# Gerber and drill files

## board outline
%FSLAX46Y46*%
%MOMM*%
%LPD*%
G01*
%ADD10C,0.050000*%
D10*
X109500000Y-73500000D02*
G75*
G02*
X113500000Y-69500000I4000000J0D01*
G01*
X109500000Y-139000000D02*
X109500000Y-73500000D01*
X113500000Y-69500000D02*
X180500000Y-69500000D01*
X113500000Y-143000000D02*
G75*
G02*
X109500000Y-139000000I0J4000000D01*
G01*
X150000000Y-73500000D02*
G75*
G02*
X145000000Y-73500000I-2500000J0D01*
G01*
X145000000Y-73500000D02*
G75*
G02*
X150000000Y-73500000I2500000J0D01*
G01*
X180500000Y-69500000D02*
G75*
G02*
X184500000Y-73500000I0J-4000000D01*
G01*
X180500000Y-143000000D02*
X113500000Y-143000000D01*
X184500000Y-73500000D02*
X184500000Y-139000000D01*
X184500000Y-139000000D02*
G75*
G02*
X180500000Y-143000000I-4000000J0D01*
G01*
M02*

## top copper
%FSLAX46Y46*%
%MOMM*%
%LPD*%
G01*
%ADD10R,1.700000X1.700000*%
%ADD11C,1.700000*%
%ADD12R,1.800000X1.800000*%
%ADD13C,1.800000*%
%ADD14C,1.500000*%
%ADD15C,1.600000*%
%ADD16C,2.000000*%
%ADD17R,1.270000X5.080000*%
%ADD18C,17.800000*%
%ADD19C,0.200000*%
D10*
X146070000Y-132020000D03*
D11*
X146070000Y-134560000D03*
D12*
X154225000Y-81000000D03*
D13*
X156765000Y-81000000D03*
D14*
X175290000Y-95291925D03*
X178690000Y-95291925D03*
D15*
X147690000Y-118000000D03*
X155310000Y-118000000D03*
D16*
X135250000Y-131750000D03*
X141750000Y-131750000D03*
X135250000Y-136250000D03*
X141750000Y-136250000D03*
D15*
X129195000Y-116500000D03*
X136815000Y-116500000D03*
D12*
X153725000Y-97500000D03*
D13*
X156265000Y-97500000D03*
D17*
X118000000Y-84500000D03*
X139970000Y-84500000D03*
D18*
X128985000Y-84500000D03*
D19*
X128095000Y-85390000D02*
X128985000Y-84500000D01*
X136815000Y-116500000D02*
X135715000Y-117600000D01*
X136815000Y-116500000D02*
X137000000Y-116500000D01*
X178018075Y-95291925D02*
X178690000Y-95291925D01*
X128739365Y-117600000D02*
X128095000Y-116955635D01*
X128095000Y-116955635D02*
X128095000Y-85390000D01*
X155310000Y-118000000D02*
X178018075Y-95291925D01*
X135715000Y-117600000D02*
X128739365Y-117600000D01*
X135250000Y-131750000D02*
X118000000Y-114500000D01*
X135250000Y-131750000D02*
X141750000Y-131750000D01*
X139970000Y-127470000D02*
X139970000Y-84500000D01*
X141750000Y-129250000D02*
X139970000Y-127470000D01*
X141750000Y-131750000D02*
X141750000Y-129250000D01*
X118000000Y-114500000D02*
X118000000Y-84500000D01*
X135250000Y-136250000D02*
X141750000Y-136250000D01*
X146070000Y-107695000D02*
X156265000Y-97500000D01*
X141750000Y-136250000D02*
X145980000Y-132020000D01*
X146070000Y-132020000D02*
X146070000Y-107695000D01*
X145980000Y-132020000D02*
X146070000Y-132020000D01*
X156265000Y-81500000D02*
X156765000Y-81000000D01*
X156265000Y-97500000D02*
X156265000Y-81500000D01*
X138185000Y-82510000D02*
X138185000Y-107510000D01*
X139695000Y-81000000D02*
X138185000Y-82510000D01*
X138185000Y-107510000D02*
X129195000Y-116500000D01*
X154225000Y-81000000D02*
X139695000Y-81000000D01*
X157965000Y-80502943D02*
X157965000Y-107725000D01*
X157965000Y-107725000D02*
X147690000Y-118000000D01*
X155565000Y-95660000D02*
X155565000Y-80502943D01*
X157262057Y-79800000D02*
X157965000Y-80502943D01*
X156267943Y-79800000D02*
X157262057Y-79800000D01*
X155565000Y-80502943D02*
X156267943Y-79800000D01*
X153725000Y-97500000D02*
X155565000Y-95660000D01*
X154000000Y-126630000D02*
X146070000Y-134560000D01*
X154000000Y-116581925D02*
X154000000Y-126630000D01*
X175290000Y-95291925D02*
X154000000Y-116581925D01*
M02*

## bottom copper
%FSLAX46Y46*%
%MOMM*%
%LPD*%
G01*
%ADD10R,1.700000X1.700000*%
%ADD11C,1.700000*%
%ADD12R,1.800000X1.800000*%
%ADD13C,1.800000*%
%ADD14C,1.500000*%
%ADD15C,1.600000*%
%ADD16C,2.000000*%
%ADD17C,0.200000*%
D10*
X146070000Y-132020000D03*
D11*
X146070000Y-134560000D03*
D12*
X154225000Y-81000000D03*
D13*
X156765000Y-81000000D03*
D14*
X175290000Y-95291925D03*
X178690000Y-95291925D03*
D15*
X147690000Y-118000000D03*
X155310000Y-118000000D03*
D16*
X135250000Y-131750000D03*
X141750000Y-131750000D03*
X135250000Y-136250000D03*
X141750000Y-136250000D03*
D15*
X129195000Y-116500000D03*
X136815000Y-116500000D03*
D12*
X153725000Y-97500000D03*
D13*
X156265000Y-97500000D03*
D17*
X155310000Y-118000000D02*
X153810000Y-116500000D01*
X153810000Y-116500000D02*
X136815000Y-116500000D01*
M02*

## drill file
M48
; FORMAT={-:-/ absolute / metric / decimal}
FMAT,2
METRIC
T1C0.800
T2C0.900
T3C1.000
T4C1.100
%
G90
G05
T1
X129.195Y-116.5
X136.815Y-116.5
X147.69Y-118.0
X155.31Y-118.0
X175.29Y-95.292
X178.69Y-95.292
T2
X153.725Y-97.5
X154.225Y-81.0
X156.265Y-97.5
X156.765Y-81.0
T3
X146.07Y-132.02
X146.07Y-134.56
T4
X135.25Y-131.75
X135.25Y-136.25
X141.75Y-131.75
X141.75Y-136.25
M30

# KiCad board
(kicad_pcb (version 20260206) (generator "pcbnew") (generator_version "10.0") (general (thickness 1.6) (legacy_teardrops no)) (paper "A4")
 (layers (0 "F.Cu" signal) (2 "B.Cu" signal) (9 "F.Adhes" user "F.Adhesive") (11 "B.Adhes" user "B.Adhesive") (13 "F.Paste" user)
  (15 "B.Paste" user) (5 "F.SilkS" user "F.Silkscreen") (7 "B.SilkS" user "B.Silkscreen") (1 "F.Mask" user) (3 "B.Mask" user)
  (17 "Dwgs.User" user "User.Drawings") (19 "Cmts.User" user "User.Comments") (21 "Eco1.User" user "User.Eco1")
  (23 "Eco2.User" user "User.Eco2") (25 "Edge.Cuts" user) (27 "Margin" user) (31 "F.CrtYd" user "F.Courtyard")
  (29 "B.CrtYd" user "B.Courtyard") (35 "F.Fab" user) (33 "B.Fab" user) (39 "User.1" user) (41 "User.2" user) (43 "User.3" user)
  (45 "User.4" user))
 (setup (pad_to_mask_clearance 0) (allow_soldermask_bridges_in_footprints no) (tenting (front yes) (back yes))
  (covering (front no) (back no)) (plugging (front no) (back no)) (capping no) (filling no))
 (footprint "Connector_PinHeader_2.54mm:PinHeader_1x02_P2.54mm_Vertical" (layer "F.Cu") (at 146.07 132.02)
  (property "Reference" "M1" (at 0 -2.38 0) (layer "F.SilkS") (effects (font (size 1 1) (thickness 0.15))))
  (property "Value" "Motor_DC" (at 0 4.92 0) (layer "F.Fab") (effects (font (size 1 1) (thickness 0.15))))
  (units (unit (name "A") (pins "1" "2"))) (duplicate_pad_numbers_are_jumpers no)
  (pad "1" thru_hole rect (at 0 0) (size 1.7 1.7) (drill 1) (layers "*.Cu" "*.Mask") (remove_unused_layers no) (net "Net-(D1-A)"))
  (pad "2" thru_hole circle (at 0 2.54) (size 1.7 1.7) (drill 1) (layers "*.Cu" "*.Mask") (remove_unused_layers no) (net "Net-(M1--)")))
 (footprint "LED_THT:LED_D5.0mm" (layer "F.Cu") (at 154.225 81)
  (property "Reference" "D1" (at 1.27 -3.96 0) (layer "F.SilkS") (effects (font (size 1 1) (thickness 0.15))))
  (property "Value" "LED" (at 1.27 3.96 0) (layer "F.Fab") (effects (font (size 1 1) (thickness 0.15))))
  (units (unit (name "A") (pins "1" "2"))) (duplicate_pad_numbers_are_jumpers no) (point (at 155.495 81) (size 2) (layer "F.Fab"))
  (pad "1" thru_hole rect (at 0 0) (size 1.8 1.8) (drill 0.9) (layers "*.Cu" "*.Mask") (remove_unused_layers no) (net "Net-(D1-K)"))
  (pad "2" thru_hole circle (at 2.54 0) (size 1.8 1.8) (drill 0.9) (layers "*.Cu" "*.Mask") (remove_unused_layers no) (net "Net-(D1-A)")))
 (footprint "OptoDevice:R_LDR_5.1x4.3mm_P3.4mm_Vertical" (layer "F.Cu") (at 175.29 95.291925)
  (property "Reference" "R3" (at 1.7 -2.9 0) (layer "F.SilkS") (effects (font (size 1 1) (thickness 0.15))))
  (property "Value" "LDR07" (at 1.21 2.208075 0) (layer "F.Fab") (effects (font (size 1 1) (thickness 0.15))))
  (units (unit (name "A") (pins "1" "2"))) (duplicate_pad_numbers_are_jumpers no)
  (pad "1" thru_hole circle (at 0 0) (size 1.5 1.5) (drill 0.8) (layers "*.Cu" "*.Mask") (remove_unused_layers no) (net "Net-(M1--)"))
  (pad "2" thru_hole circle (at 3.4 0) (size 1.5 1.5) (drill 0.8) (layers "*.Cu" "*.Mask") (remove_unused_layers no) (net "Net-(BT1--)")))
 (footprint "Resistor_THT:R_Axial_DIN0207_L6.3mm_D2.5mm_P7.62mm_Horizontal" (layer "F.Cu") (at 147.69 118)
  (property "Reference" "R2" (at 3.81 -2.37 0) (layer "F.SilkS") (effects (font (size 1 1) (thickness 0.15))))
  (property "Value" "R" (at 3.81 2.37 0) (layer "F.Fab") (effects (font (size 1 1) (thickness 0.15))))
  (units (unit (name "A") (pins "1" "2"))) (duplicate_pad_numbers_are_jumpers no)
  (pad "1" thru_hole circle (at 0 0) (size 1.6 1.6) (drill 0.8) (layers "*.Cu" "*.Mask") (remove_unused_layers no) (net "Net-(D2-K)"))
  (pad "2" thru_hole circle (at 7.62 0) (size 1.6 1.6) (drill 0.8) (layers "*.Cu" "*.Mask") (remove_unused_layers no) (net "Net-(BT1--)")))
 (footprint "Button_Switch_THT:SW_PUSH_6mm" (layer "F.Cu") (at 135.25 131.75)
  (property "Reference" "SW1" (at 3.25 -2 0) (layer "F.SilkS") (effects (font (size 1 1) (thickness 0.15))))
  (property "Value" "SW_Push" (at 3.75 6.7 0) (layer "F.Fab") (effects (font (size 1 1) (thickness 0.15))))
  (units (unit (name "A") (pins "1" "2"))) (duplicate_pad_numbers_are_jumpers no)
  (pad "1" thru_hole circle (at 0 0 90) (size 2 2) (drill 1.1) (layers "*.Cu" "*.Mask") (remove_unused_layers no) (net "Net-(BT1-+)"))
  (pad "1" thru_hole circle (at 6.5 0 90) (size 2 2) (drill 1.1) (layers "*.Cu" "*.Mask") (remove_unused_layers no) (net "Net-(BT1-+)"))
  (pad "2" thru_hole circle (at 0 4.5 90) (size 2 2) (drill 1.1) (layers "*.Cu" "*.Mask") (remove_unused_layers no) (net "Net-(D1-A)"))
  (pad "2" thru_hole circle (at 6.5 4.5 90) (size 2 2) (drill 1.1) (layers "*.Cu" "*.Mask") (remove_unused_layers no) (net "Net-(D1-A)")))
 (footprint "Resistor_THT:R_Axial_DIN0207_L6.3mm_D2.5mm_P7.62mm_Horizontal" (layer "F.Cu") (at 129.195 116.5)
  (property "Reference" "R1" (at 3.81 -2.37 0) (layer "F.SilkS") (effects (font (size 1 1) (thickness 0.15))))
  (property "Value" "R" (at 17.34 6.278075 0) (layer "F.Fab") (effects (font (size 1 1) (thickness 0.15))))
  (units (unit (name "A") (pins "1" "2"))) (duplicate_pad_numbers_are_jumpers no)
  (pad "1" thru_hole circle (at 0 0) (size 1.6 1.6) (drill 0.8) (layers "*.Cu" "*.Mask") (remove_unused_layers no) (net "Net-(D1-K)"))
  (pad "2" thru_hole circle (at 7.62 0) (size 1.6 1.6) (drill 0.8) (layers "*.Cu" "*.Mask") (remove_unused_layers no) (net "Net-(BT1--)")))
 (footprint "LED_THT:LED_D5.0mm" (layer "F.Cu") (at 153.725 97.5)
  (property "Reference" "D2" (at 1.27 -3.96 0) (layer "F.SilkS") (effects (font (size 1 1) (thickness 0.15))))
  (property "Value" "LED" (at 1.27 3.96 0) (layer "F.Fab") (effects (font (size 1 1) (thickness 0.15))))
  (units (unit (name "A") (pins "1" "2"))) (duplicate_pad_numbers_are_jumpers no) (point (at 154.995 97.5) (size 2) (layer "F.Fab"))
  (pad "1" thru_hole rect (at 0 0) (size 1.8 1.8) (drill 0.9) (layers "*.Cu" "*.Mask") (remove_unused_layers no) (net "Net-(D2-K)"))
  (pad "2" thru_hole circle (at 2.54 0) (size 1.8 1.8) (drill 0.9) (layers "*.Cu" "*.Mask") (remove_unused_layers no) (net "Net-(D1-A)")))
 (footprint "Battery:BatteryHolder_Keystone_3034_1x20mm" (layer "F.Cu") (at 128.985 84.5)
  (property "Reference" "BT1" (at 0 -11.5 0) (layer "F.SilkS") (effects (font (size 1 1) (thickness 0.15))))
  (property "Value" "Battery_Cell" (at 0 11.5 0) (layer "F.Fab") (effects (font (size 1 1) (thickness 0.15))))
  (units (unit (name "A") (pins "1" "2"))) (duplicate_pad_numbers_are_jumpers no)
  (pad "1" smd rect (at -10.985 0) (size 1.27 5.08) (layers "F.Cu" "F.Mask" "F.Paste") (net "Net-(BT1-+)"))
  (pad "1" smd rect (at 10.985 0) (size 1.27 5.08) (layers "F.Cu" "F.Mask" "F.Paste") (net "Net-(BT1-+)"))
  (pad "2" smd circle (at 0 0) (size 17.8 17.8) (layers "F.Cu" "F.Mask") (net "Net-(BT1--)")))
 (gr_arc (start 109.5 73.5) (mid 110.671573 70.671573) (end 113.5 69.5) (stroke (width 0.05) (type default)) (layer "Edge.Cuts"))
 (gr_line (start 109.5 139) (end 109.5 73.5) (stroke (width 0.05) (type default)) (layer "Edge.Cuts"))
 (gr_line (start 113.5 69.5) (end 180.5 69.5) (stroke (width 0.05) (type default)) (layer "Edge.Cuts"))
 (gr_arc (start 113.5 143) (mid 110.671573 141.828427) (end 109.5 139) (stroke (width 0.05) (type default)) (layer "Edge.Cuts"))
 (gr_circle (center 147.5 73.5) (end 149 75.5) (stroke (width 0.05) (type default)) (fill no) (layer "Edge.Cuts"))
 (gr_arc (start 180.5 69.5) (mid 183.328427 70.671573) (end 184.5 73.5) (stroke (width 0.05) (type default)) (layer "Edge.Cuts"))
 (gr_line (start 180.5 143) (end 113.5 143) (stroke (width 0.05) (type default)) (layer "Edge.Cuts"))
 (gr_line (start 184.5 73.5) (end 184.5 139) (stroke (width 0.05) (type default)) (layer "Edge.Cuts"))
 (gr_arc (start 184.5 139) (mid 183.328427 141.828427) (end 180.5 143) (stroke (width 0.05) (type default)) (layer "Edge.Cuts"))
 (segment (start 128.095 85.39) (end 128.985 84.5) (width 0.2) (layer "F.Cu") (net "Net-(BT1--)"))
 (segment (start 136.815 116.5) (end 135.715 117.6) (width 0.2) (layer "F.Cu") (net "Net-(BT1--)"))
 (segment (start 136.815 116.5) (end 137 116.5) (width 0.2) (layer "F.Cu") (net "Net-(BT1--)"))
 (segment (start 178.018075 95.291925) (end 178.69 95.291925) (width 0.2) (layer "F.Cu") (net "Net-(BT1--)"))
 (segment (start 128.739365 117.6) (end 128.095 116.955635) (width 0.2) (layer "F.Cu") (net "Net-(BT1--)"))
 (segment (start 128.095 116.955635) (end 128.095 85.39) (width 0.2) (layer "F.Cu") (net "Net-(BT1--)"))
 (segment (start 155.31 118) (end 178.018075 95.291925) (width 0.2) (layer "F.Cu") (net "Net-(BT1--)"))
 (segment (start 135.715 117.6) (end 128.739365 117.6) (width 0.2) (layer "F.Cu") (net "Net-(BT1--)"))
 (segment (start 155.31 118) (end 153.81 116.5) (width 0.2) (layer "B.Cu") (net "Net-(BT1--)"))
 (segment (start 153.81 116.5) (end 136.815 116.5) (width 0.2) (layer "B.Cu") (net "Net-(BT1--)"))
 (segment (start 135.25 131.75) (end 118 114.5) (width 0.2) (layer "F.Cu") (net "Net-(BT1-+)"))
 (segment (start 135.25 131.75) (end 141.75 131.75) (width 0.2) (layer "F.Cu") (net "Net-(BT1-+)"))
 (segment (start 139.97 127.47) (end 139.97 84.5) (width 0.2) (layer "F.Cu") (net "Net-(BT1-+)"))
 (segment (start 141.75 129.25) (end 139.97 127.47) (width 0.2) (layer "F.Cu") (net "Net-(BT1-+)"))
 (segment (start 141.75 131.75) (end 141.75 129.25) (width 0.2) (layer "F.Cu") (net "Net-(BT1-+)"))
 (segment (start 118 114.5) (end 118 84.5) (width 0.2) (layer "F.Cu") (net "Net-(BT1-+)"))
 (segment (start 135.25 136.25) (end 141.75 136.25) (width 0.2) (layer "F.Cu") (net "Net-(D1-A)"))
 (segment (start 146.07 107.695) (end 156.265 97.5) (width 0.2) (layer "F.Cu") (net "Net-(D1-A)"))
 (segment (start 141.75 136.25) (end 145.98 132.02) (width 0.2) (layer "F.Cu") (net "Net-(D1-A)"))
 (segment (start 146.07 132.02) (end 146.07 107.695) (width 0.2) (layer "F.Cu") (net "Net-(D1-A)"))
 (segment (start 145.98 132.02) (end 146.07 132.02) (width 0.2) (layer "F.Cu") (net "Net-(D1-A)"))
 (segment (start 156.265 81.5) (end 156.765 81) (width 0.2) (layer "F.Cu") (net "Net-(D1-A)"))
 (segment (start 156.265 97.5) (end 156.265 81.5) (width 0.2) (layer "F.Cu") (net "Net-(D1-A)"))
 (segment (start 138.185 82.51) (end 138.185 107.51) (width 0.2) (layer "F.Cu") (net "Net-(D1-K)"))
 (segment (start 139.695 81) (end 138.185 82.51) (width 0.2) (layer "F.Cu") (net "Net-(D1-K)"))
 (segment (start 138.185 107.51) (end 129.195 116.5) (width 0.2) (layer "F.Cu") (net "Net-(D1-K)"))
 (segment (start 154.225 81) (end 139.695 81) (width 0.2) (layer "F.Cu") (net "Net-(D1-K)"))
 (segment (start 157.965 80.502943) (end 157.965 107.725) (width 0.2) (layer "F.Cu") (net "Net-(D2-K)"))
 (segment (start 157.965 107.725) (end 147.69 118) (width 0.2) (layer "F.Cu") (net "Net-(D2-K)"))
 (segment (start 155.565 95.66) (end 155.565 80.502943) (width 0.2) (layer "F.Cu") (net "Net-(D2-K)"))
 (segment (start 157.262057 79.8) (end 157.965 80.502943) (width 0.2) (layer "F.Cu") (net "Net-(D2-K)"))
 (segment (start 156.267943 79.8) (end 157.262057 79.8) (width 0.2) (layer "F.Cu") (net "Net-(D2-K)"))
 (segment (start 155.565 80.502943) (end 156.267943 79.8) (width 0.2) (layer "F.Cu") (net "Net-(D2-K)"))
 (segment (start 153.725 97.5) (end 155.565 95.66) (width 0.2) (layer "F.Cu") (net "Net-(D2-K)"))
 (segment (start 154 126.63) (end 146.07 134.56) (width 0.2) (layer "F.Cu") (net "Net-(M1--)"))
 (segment (start 154 116.581925) (end 154 126.63) (width 0.2) (layer "F.Cu") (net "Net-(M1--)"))
 (segment (start 175.29 95.291925) (end 154 116.581925) (width 0.2) (layer "F.Cu") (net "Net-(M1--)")))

